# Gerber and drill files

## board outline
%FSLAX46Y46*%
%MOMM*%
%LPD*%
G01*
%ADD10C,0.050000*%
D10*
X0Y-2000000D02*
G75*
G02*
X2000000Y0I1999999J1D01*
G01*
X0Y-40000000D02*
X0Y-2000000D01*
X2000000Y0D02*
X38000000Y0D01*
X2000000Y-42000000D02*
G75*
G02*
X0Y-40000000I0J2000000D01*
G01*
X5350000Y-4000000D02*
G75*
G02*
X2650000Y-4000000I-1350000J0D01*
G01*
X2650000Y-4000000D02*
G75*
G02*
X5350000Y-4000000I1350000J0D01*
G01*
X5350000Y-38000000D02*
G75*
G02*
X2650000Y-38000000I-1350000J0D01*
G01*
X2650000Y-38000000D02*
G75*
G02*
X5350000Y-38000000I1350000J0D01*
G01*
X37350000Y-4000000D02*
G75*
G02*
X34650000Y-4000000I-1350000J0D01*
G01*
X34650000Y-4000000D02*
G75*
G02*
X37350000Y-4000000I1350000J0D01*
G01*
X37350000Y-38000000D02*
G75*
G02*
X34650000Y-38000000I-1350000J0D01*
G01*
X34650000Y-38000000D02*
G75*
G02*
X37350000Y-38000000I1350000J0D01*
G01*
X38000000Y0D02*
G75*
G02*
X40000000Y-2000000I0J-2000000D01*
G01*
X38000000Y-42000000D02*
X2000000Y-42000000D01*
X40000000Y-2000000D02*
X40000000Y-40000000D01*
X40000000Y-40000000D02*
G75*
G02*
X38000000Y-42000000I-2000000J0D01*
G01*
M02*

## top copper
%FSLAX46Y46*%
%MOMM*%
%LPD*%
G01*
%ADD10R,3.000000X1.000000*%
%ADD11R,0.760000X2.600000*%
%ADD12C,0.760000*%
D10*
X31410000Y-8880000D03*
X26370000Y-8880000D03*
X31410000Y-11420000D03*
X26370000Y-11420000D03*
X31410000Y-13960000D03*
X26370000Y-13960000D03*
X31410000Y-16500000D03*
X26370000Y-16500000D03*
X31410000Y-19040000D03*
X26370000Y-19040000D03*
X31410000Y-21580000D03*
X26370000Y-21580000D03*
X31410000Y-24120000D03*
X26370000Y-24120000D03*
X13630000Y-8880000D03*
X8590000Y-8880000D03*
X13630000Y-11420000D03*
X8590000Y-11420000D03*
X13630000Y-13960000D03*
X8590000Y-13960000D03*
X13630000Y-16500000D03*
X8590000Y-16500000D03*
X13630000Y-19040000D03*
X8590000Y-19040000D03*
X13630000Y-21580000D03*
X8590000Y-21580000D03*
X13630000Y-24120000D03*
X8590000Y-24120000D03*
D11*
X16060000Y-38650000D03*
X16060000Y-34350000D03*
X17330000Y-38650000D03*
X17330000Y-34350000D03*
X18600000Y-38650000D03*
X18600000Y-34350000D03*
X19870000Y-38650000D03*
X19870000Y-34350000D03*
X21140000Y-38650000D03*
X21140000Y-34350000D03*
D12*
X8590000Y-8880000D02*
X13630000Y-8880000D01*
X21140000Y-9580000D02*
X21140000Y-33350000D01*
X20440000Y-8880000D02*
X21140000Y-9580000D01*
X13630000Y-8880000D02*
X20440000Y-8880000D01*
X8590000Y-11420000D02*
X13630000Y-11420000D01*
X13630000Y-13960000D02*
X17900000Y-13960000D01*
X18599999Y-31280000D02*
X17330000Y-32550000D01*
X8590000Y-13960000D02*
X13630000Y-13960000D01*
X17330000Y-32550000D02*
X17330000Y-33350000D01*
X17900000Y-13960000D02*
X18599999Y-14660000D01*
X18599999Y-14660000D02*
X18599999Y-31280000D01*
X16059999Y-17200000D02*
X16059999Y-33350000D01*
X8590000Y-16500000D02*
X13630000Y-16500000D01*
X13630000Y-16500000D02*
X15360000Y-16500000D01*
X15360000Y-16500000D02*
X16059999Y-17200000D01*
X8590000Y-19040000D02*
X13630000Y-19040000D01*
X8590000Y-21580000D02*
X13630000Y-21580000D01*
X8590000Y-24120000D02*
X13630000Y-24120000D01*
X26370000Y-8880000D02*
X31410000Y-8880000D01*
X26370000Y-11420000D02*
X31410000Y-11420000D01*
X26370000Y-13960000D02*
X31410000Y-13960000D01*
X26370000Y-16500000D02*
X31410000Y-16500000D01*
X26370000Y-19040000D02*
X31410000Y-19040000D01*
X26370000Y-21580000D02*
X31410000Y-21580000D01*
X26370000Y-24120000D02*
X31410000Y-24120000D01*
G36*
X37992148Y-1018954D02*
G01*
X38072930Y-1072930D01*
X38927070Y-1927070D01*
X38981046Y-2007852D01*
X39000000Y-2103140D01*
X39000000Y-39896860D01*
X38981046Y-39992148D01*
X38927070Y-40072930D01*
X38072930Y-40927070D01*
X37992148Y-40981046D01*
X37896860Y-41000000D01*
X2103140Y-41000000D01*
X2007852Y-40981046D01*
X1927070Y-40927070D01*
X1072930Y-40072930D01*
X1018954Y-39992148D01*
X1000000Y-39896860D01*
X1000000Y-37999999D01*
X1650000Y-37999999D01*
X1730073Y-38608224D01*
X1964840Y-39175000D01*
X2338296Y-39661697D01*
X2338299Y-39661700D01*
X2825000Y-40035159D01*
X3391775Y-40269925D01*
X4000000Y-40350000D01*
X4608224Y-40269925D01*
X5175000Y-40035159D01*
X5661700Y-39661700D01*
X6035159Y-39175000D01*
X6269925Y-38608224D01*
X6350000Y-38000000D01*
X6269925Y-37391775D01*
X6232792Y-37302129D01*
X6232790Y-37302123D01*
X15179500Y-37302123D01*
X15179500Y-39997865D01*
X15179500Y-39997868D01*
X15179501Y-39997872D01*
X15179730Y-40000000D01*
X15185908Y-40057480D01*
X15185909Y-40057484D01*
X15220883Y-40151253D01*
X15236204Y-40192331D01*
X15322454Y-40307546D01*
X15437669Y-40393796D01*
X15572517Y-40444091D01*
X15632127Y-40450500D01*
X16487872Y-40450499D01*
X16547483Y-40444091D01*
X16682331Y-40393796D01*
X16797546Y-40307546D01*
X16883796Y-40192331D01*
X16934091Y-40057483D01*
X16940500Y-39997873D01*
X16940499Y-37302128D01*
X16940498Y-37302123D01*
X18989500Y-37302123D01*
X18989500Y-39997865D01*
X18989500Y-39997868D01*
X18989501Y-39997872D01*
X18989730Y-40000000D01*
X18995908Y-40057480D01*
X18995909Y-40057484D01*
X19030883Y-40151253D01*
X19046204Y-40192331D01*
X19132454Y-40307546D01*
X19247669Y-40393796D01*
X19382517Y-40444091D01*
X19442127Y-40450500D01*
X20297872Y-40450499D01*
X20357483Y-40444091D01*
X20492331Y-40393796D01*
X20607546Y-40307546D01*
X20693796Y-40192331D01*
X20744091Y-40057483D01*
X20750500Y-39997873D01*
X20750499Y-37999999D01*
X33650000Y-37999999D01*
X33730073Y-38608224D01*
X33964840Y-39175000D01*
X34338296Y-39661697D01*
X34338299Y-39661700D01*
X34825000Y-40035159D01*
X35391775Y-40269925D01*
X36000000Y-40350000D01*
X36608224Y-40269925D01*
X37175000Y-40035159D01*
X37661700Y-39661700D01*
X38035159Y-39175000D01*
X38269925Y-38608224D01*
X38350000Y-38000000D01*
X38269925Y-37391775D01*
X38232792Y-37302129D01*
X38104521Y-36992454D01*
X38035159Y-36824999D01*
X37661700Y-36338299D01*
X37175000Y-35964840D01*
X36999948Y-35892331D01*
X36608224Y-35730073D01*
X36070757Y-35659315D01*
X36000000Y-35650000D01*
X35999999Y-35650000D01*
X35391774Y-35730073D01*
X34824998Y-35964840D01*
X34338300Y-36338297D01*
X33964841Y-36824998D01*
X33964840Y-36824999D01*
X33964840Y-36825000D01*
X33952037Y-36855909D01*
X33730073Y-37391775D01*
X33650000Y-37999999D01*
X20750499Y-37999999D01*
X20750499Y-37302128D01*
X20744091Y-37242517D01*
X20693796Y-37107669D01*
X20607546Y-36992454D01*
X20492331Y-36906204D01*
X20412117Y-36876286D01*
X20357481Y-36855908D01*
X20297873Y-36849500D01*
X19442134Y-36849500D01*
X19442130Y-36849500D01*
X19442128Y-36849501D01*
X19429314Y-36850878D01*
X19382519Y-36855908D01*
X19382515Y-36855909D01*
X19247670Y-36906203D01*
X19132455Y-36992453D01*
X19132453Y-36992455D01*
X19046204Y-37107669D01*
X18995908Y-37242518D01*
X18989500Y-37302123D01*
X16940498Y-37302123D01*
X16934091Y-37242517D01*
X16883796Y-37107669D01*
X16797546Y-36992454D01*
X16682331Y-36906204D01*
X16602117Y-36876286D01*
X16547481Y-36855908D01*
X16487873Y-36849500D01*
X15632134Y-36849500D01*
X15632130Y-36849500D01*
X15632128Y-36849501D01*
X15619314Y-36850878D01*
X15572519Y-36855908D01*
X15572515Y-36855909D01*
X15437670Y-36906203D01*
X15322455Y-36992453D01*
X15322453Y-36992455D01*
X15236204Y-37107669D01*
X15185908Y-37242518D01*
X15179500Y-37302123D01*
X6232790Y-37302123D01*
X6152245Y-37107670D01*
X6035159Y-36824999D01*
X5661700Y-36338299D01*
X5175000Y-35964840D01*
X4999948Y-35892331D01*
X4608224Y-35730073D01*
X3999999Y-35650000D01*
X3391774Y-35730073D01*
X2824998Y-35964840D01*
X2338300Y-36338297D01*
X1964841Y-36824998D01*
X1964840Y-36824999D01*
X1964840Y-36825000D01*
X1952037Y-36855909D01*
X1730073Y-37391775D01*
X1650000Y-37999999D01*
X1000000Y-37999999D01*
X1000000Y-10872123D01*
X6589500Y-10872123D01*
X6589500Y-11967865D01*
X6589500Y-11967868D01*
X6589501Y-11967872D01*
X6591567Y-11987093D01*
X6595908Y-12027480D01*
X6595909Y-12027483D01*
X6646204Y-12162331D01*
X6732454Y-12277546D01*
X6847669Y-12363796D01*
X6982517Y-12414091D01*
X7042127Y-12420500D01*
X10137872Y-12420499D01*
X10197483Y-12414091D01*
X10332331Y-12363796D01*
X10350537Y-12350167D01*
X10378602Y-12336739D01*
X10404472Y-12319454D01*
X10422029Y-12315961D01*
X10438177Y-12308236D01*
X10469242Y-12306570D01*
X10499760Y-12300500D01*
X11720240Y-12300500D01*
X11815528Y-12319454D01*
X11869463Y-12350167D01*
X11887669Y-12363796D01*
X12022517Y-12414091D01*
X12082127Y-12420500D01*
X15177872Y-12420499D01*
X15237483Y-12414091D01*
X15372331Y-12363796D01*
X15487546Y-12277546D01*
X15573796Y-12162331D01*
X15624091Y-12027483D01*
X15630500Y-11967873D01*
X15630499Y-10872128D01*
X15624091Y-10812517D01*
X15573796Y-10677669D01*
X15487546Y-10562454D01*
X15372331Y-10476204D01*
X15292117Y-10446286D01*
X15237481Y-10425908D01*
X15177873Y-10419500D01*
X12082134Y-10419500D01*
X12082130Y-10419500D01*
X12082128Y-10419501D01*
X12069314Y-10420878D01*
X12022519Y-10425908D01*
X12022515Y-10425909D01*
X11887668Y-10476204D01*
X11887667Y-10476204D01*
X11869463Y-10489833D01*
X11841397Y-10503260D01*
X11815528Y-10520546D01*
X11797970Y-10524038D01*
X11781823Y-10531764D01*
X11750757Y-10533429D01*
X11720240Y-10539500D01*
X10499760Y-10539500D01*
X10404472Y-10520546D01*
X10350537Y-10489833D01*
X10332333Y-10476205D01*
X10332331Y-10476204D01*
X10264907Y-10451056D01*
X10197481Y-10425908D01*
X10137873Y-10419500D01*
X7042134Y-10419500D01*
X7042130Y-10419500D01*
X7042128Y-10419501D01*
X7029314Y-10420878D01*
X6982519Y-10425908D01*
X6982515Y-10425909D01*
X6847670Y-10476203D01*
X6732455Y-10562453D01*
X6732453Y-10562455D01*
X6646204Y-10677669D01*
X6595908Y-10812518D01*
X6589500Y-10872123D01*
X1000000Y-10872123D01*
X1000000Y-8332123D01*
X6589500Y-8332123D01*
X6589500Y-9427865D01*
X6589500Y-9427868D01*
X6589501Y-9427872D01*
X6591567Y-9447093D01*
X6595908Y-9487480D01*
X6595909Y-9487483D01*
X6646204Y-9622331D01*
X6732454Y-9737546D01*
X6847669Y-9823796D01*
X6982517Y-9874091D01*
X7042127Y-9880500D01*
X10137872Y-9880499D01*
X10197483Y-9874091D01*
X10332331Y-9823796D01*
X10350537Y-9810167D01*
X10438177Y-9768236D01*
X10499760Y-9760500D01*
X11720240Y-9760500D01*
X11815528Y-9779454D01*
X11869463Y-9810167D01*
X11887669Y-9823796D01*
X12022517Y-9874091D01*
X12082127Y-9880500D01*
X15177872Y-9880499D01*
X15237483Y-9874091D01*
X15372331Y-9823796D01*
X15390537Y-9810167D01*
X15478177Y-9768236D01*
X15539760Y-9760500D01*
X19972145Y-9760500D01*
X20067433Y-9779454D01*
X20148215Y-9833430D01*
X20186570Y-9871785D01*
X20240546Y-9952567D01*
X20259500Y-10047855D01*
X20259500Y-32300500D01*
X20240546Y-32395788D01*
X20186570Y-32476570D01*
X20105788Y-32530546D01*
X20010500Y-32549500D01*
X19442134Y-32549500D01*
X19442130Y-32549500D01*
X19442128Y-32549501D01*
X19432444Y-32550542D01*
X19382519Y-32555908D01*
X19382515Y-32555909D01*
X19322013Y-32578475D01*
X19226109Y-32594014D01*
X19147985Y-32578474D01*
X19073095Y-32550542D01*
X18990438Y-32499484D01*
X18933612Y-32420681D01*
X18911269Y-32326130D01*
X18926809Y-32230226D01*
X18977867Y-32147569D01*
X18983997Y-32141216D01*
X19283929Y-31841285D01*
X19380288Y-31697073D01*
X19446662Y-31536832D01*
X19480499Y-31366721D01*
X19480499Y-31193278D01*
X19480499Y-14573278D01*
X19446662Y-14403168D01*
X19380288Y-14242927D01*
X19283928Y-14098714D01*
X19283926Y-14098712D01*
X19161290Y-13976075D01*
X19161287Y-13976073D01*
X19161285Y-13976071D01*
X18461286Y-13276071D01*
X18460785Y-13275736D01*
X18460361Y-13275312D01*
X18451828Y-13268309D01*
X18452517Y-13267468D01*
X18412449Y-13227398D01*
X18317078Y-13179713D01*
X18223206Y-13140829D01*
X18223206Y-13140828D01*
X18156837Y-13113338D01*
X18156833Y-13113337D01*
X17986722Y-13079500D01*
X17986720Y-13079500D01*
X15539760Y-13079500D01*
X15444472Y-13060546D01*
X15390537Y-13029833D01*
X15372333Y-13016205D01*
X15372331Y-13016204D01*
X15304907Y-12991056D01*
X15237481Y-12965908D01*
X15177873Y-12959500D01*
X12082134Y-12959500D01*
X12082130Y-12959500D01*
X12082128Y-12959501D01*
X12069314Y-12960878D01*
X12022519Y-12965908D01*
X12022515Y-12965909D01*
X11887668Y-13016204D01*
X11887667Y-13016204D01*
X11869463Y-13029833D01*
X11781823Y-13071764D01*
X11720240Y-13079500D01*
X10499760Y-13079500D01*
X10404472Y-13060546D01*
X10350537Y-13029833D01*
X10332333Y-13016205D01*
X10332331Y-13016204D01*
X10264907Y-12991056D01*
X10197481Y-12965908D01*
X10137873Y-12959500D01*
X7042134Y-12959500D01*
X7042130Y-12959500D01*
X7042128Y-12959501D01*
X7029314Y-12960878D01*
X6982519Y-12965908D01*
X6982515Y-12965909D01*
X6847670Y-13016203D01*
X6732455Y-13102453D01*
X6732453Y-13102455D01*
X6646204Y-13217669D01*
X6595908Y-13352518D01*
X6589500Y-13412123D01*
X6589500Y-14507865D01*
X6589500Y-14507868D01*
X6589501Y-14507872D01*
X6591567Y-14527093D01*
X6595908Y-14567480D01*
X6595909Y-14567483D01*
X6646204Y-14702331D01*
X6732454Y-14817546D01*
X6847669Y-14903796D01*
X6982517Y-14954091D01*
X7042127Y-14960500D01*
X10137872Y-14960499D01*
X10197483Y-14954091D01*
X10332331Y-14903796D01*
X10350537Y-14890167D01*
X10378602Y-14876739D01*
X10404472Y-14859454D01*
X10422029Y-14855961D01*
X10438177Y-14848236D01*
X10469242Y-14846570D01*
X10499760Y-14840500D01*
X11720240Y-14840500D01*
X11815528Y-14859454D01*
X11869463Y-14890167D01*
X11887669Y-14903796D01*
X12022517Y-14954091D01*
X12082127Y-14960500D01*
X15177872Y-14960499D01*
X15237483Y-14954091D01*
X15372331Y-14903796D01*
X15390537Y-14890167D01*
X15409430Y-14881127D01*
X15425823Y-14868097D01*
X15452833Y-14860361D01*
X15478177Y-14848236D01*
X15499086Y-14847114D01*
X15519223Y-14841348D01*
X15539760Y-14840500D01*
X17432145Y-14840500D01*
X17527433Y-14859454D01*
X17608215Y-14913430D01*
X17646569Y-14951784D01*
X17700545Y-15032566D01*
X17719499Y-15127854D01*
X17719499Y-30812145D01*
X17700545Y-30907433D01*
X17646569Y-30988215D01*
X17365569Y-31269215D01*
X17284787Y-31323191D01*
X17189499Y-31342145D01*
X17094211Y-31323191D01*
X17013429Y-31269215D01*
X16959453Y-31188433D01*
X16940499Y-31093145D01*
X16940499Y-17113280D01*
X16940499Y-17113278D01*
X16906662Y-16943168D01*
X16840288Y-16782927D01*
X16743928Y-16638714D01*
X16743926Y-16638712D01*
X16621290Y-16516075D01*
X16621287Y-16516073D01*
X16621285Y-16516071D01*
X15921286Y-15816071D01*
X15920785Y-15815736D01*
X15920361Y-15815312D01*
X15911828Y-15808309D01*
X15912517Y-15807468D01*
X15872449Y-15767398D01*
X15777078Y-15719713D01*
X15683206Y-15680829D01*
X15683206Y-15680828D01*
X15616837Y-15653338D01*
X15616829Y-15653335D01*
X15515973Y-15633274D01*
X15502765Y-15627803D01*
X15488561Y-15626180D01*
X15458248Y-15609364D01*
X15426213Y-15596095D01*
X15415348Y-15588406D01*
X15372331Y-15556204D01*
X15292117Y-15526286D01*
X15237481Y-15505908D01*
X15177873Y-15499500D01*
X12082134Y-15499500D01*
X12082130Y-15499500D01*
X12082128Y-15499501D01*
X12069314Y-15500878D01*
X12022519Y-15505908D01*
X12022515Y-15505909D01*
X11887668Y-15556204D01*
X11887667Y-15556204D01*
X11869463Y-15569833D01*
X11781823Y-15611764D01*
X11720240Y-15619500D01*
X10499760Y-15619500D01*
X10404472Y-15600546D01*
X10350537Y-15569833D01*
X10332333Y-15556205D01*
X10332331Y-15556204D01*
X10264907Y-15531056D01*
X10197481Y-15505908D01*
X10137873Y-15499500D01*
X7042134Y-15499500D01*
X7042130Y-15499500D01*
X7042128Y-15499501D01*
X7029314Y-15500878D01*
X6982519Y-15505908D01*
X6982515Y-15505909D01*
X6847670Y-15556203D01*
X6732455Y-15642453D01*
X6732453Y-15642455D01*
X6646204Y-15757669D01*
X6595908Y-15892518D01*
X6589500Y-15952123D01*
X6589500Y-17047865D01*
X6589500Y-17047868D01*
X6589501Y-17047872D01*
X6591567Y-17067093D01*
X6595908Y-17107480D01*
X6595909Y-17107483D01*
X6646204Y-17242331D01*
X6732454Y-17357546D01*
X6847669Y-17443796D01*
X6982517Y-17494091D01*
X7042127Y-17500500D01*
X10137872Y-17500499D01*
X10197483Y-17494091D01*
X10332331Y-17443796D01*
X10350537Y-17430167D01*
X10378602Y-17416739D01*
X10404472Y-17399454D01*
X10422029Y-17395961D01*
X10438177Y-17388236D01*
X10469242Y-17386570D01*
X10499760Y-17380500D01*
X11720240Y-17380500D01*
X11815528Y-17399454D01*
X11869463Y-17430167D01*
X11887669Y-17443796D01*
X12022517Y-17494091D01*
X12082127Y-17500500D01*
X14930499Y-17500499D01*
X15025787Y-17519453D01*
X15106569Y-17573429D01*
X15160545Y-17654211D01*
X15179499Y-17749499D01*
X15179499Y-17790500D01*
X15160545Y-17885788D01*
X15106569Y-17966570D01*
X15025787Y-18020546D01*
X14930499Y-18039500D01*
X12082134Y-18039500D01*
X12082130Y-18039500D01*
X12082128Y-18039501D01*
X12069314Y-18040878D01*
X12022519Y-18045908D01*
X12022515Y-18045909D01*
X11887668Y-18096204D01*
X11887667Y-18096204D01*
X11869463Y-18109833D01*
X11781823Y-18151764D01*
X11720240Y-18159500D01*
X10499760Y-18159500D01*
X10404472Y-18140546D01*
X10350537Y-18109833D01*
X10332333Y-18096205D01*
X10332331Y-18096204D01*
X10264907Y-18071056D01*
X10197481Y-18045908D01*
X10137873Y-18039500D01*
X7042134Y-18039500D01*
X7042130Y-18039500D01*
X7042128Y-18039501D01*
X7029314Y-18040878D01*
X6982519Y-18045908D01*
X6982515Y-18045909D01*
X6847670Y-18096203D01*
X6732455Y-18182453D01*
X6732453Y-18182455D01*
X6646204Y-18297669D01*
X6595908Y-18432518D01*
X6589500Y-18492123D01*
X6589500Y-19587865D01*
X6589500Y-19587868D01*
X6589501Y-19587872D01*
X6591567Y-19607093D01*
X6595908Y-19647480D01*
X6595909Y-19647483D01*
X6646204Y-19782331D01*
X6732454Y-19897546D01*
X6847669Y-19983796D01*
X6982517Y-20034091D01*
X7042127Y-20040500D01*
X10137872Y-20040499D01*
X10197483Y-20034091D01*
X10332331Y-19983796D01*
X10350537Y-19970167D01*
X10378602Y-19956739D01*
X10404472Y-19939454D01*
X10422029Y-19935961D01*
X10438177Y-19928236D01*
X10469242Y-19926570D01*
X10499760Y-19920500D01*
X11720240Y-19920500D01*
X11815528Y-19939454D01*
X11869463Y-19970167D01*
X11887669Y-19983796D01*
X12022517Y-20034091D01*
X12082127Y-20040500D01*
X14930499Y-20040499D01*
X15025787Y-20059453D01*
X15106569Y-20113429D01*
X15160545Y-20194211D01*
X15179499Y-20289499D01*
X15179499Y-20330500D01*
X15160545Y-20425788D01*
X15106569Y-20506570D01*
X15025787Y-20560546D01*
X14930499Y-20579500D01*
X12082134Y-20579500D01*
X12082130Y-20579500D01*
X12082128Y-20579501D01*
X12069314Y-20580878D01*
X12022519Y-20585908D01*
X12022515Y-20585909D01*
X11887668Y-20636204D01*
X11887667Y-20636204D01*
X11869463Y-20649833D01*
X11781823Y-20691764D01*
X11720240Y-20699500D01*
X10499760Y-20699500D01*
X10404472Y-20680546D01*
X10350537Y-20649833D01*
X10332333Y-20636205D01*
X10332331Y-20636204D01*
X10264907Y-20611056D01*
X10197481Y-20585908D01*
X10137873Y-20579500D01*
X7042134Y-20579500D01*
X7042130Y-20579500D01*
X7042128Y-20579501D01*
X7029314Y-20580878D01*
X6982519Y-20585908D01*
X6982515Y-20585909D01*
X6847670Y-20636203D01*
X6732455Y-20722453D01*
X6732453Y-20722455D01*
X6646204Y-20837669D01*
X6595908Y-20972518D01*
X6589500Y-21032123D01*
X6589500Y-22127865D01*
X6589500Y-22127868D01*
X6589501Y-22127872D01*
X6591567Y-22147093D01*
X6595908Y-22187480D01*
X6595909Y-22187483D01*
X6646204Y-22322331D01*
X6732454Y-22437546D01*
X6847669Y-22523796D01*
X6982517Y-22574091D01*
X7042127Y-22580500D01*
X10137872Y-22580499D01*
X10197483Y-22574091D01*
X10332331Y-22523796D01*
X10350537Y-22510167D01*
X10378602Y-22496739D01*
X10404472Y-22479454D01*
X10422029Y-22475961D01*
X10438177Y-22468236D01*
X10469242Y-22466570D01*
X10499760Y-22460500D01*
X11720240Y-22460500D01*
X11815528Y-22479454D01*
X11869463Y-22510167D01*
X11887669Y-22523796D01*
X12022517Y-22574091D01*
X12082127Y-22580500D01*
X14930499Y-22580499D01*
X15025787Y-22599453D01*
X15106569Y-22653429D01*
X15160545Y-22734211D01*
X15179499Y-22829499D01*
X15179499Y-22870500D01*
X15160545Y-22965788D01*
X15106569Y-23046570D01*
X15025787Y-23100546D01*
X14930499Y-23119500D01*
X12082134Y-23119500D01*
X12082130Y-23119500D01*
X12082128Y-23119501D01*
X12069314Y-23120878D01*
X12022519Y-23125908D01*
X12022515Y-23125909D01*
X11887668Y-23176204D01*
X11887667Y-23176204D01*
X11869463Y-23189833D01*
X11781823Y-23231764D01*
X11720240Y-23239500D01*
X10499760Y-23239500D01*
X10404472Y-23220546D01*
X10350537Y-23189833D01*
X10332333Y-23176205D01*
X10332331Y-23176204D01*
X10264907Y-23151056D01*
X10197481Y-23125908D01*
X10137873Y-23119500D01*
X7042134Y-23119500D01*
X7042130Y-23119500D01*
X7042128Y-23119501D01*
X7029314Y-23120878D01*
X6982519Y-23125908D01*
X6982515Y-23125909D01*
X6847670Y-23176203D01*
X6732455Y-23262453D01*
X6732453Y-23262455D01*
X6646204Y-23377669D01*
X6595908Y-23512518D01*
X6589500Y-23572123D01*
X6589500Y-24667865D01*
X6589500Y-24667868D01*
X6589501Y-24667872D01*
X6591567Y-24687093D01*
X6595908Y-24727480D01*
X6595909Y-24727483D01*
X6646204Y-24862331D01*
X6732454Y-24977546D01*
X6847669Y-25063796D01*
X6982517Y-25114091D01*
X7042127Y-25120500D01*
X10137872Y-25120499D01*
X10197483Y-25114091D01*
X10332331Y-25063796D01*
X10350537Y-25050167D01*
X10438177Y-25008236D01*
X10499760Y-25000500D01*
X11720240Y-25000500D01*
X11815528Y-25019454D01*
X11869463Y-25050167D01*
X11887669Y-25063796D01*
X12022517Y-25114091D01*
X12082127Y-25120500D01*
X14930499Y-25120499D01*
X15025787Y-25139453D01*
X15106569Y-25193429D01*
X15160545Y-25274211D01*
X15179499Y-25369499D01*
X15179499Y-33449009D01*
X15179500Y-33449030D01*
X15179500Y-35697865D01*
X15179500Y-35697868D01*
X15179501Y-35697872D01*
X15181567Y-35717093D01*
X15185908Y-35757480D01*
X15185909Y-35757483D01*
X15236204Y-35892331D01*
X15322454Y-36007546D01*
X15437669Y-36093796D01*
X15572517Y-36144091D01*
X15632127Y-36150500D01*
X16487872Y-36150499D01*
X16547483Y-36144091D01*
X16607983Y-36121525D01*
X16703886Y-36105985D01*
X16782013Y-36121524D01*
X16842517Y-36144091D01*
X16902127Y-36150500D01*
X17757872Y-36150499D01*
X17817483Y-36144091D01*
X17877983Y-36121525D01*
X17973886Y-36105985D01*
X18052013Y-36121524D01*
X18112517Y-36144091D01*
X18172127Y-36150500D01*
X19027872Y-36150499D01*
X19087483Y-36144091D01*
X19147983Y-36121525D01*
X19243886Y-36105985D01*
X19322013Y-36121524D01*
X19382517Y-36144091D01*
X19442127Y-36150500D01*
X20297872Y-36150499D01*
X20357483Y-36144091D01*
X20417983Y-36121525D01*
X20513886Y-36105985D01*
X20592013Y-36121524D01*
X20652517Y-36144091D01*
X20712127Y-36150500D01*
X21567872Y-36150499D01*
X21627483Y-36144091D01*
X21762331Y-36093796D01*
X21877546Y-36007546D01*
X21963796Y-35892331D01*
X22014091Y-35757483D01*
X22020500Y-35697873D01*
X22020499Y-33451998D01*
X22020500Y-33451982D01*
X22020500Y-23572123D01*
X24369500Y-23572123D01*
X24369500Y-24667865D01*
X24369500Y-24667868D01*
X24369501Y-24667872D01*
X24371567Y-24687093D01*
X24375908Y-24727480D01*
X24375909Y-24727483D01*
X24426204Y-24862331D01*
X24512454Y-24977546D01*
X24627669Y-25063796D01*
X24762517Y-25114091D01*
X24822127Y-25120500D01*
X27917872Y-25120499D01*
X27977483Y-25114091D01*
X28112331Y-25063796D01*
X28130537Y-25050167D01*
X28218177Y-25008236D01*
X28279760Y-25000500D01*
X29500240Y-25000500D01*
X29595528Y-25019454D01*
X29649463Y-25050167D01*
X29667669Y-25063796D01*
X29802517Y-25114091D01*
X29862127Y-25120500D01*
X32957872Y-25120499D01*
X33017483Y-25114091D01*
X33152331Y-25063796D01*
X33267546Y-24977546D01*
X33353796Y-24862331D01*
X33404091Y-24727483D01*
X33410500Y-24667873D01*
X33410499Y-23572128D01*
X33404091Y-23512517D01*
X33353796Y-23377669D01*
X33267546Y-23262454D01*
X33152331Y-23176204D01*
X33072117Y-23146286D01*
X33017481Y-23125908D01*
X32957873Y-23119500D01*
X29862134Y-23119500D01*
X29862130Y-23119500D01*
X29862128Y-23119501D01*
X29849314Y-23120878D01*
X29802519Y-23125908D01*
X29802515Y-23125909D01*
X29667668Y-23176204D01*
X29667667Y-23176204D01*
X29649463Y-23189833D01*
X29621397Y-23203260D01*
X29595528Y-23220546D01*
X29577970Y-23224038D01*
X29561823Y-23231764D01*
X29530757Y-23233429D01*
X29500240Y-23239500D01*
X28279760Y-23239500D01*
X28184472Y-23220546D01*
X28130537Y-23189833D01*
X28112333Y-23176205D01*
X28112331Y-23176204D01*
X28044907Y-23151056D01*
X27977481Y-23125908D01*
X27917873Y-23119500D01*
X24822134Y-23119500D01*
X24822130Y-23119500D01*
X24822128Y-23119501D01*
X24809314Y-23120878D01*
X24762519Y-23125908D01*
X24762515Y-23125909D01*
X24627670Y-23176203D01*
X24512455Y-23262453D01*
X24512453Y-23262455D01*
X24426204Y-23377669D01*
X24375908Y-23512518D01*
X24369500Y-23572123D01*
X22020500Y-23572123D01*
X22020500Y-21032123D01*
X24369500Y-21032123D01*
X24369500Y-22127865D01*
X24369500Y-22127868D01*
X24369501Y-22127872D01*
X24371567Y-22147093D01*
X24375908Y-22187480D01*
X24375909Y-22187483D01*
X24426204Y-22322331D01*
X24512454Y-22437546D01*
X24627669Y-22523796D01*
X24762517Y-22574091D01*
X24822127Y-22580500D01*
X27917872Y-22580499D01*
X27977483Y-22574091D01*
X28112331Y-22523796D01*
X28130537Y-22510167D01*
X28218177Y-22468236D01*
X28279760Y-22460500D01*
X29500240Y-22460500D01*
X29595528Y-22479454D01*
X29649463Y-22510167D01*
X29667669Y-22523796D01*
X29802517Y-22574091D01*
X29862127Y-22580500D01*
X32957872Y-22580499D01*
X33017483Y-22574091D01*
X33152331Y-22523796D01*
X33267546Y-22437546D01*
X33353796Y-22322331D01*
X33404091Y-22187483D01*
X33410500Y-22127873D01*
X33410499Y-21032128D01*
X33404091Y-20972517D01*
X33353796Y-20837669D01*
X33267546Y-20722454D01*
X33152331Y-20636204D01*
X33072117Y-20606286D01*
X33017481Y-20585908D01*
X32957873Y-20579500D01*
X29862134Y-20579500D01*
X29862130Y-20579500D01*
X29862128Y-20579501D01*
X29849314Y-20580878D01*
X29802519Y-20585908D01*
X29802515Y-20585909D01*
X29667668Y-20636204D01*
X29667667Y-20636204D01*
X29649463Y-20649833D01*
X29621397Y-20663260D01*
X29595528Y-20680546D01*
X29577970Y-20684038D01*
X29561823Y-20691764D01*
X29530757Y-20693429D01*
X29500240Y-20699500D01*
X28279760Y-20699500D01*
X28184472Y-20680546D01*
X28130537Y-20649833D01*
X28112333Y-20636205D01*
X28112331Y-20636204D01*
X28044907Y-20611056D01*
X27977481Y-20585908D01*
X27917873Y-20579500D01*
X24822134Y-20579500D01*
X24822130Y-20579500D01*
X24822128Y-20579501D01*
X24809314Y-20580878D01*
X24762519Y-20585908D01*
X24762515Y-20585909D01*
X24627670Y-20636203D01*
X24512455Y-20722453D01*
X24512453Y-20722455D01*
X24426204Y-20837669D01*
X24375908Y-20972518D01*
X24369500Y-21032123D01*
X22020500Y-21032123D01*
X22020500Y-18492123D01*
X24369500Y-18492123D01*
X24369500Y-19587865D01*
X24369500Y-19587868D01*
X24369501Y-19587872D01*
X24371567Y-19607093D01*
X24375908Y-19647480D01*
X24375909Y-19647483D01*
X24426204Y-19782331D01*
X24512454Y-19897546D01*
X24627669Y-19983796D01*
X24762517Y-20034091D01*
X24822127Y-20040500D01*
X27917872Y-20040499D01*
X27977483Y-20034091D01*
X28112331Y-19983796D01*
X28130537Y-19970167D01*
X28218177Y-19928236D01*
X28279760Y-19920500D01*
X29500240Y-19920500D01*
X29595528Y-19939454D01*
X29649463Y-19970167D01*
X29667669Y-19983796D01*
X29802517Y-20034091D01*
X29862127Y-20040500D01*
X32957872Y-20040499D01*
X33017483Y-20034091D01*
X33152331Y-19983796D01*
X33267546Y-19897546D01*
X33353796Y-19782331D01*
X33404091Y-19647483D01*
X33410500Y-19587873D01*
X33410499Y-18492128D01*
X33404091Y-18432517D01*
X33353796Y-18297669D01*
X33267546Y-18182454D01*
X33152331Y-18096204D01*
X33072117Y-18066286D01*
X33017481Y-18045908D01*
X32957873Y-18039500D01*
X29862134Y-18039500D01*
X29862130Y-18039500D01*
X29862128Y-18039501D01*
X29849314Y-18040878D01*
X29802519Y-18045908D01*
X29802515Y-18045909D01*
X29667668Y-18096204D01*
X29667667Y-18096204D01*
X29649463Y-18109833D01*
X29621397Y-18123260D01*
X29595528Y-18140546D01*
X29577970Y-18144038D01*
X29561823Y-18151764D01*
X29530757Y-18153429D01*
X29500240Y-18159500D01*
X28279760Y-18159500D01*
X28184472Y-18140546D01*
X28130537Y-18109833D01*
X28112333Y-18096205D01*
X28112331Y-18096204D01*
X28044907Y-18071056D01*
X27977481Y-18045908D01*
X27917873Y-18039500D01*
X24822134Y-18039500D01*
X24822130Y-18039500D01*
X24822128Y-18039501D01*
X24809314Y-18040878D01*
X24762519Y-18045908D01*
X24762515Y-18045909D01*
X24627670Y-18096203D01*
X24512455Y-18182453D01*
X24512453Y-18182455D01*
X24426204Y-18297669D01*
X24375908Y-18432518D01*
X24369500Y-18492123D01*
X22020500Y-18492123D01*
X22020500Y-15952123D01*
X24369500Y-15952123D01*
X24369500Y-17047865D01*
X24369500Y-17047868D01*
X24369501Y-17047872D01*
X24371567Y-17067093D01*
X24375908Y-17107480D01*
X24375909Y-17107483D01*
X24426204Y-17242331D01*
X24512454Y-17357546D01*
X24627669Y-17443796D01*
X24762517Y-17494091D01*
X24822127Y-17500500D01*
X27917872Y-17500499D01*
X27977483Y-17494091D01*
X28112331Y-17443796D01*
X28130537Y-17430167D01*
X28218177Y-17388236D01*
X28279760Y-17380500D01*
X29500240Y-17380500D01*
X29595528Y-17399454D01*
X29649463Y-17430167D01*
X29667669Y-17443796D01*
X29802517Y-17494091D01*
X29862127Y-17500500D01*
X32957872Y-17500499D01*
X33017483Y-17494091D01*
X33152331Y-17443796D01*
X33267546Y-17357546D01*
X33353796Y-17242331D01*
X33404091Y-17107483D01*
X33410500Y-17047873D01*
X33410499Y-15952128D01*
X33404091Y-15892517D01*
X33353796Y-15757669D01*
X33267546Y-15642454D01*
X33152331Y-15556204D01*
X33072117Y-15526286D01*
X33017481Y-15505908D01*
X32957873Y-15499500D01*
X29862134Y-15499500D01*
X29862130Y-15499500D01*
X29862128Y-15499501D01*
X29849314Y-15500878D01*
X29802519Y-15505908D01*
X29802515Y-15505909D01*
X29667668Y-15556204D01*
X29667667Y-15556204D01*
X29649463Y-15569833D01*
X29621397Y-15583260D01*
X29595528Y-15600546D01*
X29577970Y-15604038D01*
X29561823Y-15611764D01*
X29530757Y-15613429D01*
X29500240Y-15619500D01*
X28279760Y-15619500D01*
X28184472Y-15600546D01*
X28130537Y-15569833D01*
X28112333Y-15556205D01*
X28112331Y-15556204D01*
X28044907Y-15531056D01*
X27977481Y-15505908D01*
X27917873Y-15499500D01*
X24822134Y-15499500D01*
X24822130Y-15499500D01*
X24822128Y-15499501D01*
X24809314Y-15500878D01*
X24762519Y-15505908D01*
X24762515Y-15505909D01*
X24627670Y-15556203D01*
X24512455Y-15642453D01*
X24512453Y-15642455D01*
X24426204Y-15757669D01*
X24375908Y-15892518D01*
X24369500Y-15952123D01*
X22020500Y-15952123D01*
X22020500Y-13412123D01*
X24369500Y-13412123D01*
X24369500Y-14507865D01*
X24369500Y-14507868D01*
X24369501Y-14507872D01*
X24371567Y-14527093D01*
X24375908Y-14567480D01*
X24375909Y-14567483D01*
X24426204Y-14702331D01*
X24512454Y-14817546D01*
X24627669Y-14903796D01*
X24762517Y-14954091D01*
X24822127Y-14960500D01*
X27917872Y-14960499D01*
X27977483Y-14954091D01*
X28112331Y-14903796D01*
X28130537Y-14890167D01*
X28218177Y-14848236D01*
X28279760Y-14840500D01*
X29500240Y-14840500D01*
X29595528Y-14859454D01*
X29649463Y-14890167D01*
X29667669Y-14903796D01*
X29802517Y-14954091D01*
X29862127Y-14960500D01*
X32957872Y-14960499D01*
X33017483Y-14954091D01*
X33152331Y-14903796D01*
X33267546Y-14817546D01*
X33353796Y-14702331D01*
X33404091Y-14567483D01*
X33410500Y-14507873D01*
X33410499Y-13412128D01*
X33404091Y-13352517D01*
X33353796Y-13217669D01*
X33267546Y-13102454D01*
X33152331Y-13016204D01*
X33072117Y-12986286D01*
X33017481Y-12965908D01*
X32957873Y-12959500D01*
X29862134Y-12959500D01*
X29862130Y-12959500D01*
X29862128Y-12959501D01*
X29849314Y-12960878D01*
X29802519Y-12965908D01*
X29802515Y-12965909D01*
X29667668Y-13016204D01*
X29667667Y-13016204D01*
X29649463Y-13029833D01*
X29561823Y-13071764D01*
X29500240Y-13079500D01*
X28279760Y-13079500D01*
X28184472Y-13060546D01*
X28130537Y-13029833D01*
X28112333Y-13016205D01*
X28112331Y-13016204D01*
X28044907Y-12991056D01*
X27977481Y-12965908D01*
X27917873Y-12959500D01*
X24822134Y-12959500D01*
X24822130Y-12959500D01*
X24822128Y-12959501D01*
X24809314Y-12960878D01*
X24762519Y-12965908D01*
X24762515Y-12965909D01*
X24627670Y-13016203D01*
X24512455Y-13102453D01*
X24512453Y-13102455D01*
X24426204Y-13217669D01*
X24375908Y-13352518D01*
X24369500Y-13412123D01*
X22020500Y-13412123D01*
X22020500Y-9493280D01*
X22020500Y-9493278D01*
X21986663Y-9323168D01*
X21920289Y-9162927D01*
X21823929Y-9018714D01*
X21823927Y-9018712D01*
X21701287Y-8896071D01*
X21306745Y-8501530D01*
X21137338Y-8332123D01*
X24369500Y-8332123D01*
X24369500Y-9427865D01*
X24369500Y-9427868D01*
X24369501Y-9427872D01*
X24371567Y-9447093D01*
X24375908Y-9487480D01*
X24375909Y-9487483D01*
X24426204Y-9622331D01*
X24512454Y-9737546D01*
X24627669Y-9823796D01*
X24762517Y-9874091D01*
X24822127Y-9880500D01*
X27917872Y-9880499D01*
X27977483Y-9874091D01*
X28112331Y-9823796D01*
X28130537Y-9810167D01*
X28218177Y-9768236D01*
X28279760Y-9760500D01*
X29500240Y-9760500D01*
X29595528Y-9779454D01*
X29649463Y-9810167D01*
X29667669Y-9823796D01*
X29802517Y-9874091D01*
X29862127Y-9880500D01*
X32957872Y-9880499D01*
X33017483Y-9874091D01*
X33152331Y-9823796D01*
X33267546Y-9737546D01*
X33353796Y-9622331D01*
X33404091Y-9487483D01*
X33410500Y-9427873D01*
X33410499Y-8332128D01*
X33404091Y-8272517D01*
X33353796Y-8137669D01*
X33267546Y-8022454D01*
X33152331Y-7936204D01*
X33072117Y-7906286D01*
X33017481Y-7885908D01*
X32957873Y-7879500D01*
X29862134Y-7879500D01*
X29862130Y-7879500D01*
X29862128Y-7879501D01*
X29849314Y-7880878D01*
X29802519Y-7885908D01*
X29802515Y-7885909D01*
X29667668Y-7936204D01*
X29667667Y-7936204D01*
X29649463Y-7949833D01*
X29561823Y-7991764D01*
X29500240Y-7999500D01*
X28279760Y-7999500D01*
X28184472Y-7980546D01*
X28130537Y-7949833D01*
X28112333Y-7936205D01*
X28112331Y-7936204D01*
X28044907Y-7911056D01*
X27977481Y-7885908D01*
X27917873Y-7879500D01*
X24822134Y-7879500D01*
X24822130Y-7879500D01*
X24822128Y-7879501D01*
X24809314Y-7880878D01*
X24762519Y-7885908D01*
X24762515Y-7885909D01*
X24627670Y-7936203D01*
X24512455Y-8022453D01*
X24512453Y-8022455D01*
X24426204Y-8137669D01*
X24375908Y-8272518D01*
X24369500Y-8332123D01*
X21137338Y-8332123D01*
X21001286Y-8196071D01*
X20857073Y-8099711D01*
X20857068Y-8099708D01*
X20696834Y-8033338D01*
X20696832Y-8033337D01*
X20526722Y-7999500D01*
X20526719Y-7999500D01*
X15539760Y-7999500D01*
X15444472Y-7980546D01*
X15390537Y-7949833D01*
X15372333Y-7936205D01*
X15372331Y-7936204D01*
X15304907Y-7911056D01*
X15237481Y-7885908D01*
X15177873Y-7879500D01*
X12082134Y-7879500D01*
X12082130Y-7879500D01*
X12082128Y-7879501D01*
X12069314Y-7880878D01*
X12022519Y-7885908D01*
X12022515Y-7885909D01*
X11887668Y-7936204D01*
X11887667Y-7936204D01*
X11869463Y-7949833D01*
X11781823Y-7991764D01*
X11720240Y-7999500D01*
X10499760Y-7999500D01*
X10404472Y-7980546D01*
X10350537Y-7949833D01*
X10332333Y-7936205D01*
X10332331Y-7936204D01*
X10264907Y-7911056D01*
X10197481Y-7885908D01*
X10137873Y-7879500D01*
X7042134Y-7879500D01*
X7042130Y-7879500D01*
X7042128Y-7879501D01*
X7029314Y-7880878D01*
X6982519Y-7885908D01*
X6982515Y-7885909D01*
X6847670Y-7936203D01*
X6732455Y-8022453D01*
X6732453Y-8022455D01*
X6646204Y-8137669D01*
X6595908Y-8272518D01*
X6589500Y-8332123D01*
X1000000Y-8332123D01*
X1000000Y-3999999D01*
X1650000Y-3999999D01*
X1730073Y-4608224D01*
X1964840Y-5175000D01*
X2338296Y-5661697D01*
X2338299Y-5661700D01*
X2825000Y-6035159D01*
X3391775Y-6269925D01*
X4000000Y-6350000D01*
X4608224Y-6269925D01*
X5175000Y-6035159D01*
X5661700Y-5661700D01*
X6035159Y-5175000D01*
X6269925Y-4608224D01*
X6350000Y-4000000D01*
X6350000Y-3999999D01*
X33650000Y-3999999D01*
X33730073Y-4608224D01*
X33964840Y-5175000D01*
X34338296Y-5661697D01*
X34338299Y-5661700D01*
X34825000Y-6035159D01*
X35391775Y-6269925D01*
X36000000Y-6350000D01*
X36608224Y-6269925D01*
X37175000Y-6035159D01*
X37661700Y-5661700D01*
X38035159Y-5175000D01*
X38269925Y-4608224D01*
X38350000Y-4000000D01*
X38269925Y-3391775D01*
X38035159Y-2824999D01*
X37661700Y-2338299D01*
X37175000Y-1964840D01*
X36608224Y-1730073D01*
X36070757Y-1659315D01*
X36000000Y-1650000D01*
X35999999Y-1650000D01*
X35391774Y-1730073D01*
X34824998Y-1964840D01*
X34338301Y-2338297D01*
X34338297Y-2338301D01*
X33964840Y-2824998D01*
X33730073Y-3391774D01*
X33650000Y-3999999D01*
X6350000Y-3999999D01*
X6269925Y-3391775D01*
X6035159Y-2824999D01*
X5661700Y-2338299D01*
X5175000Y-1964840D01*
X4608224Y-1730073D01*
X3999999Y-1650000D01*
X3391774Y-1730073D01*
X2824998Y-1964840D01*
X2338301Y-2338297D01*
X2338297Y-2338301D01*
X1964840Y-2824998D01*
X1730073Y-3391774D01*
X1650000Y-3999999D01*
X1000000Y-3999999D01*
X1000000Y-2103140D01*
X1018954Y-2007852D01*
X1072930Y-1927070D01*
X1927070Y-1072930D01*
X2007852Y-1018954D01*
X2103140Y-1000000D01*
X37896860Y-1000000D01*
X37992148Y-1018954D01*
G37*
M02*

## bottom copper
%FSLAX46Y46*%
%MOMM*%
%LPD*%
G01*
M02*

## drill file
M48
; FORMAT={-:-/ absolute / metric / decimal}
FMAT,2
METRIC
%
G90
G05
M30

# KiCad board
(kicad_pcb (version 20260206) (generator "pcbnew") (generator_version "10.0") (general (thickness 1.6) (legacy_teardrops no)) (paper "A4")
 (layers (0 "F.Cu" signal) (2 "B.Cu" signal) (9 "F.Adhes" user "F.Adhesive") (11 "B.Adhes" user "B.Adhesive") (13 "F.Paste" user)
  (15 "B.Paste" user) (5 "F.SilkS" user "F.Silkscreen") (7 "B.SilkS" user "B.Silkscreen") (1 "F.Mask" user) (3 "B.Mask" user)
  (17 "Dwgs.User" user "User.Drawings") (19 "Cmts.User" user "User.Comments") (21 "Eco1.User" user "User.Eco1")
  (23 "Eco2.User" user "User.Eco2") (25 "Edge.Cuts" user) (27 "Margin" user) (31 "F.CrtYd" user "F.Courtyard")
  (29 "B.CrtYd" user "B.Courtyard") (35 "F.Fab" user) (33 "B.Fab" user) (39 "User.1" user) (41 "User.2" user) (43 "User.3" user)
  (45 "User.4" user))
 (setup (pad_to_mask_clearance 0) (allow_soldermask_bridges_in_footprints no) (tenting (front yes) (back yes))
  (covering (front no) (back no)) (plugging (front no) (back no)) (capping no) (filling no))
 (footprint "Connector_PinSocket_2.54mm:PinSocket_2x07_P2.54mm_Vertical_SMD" (layer "F.Cu") (at 28.89 16.5)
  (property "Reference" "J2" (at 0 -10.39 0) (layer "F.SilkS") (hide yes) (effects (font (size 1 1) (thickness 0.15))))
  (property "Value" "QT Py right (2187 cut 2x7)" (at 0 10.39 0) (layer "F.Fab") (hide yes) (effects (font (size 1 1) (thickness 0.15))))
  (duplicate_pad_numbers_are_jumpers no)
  (pad "1" smd rect (at 2.52 -7.62) (size 3 1) (layers "F.Cu" "F.Mask" "F.Paste") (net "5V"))
  (pad "2" smd rect (at -2.52 -7.62) (size 3 1) (layers "F.Cu" "F.Mask" "F.Paste") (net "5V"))
  (pad "3" smd rect (at 2.52 -5.08) (size 3 1) (layers "F.Cu" "F.Mask" "F.Paste") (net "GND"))
  (pad "4" smd rect (at -2.52 -5.08) (size 3 1) (layers "F.Cu" "F.Mask" "F.Paste") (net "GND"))
  (pad "5" smd rect (at 2.52 -2.54) (size 3 1) (layers "F.Cu" "F.Mask" "F.Paste") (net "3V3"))
  (pad "6" smd rect (at -2.52 -2.54) (size 3 1) (layers "F.Cu" "F.Mask" "F.Paste") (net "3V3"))
  (pad "7" smd rect (at 2.52 0) (size 3 1) (layers "F.Cu" "F.Mask" "F.Paste") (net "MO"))
  (pad "8" smd rect (at -2.52 0) (size 3 1) (layers "F.Cu" "F.Mask" "F.Paste") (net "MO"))
  (pad "9" smd rect (at 2.52 2.54) (size 3 1) (layers "F.Cu" "F.Mask" "F.Paste") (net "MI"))
  (pad "10" smd rect (at -2.52 2.54) (size 3 1) (layers "F.Cu" "F.Mask" "F.Paste") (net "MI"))
  (pad "11" smd rect (at 2.52 5.08) (size 3 1) (layers "F.Cu" "F.Mask" "F.Paste") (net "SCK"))
  (pad "12" smd rect (at -2.52 5.08) (size 3 1) (layers "F.Cu" "F.Mask" "F.Paste") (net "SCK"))
  (pad "13" smd rect (at 2.52 7.62) (size 3 1) (layers "F.Cu" "F.Mask" "F.Paste") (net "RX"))
  (pad "14" smd rect (at -2.52 7.62) (size 3 1) (layers "F.Cu" "F.Mask" "F.Paste") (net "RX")))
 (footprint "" (layer "F.Cu") (at 11.11 26.851)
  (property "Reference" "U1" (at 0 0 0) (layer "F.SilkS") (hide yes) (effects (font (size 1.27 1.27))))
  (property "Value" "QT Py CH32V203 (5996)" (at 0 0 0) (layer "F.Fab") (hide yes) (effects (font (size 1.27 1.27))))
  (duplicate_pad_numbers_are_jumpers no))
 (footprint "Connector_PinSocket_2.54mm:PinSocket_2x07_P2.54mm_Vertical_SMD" (layer "F.Cu") (at 11.11 16.5)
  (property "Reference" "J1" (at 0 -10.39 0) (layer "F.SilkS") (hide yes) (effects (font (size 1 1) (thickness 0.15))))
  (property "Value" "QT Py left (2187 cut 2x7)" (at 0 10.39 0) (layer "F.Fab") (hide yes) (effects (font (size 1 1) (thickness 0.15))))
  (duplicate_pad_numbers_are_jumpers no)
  (pad "1" smd rect (at 2.52 -7.62) (size 3 1) (layers "F.Cu" "F.Mask" "F.Paste") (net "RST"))
  (pad "2" smd rect (at -2.52 -7.62) (size 3 1) (layers "F.Cu" "F.Mask" "F.Paste") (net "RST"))
  (pad "3" smd rect (at 2.52 -5.08) (size 3 1) (layers "F.Cu" "F.Mask" "F.Paste") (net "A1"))
  (pad "4" smd rect (at -2.52 -5.08) (size 3 1) (layers "F.Cu" "F.Mask" "F.Paste") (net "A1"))
  (pad "5" smd rect (at 2.52 -2.54) (size 3 1) (layers "F.Cu" "F.Mask" "F.Paste") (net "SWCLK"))
  (pad "6" smd rect (at -2.52 -2.54) (size 3 1) (layers "F.Cu" "F.Mask" "F.Paste") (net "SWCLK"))
  (pad "7" smd rect (at 2.52 0) (size 3 1) (layers "F.Cu" "F.Mask" "F.Paste") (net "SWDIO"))
  (pad "8" smd rect (at -2.52 0) (size 3 1) (layers "F.Cu" "F.Mask" "F.Paste") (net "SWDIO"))
  (pad "9" smd rect (at 2.52 2.54) (size 3 1) (layers "F.Cu" "F.Mask" "F.Paste") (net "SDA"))
  (pad "10" smd rect (at -2.52 2.54) (size 3 1) (layers "F.Cu" "F.Mask" "F.Paste") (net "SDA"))
  (pad "11" smd rect (at 2.52 5.08) (size 3 1) (layers "F.Cu" "F.Mask" "F.Paste") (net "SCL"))
  (pad "12" smd rect (at -2.52 5.08) (size 3 1) (layers "F.Cu" "F.Mask" "F.Paste") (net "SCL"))
  (pad "13" smd rect (at 2.52 7.62) (size 3 1) (layers "F.Cu" "F.Mask" "F.Paste") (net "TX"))
  (pad "14" smd rect (at -2.52 7.62) (size 3 1) (layers "F.Cu" "F.Mask" "F.Paste") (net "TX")))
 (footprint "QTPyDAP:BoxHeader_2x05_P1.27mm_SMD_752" (layer "F.Cu") (at 18.6 36.5 90)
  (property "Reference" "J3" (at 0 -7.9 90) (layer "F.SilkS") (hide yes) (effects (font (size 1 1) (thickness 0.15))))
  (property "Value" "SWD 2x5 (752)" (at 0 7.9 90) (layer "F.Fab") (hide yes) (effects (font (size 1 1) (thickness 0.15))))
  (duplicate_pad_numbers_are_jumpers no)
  (pad "1" smd rect (at -2.15 -2.54 90) (size 2.6 0.76) (layers "F.Cu" "F.Mask" "F.Paste"))
  (pad "2" smd rect (at 2.15 -2.54 90) (size 2.6 0.76) (layers "F.Cu" "F.Mask" "F.Paste") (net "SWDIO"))
  (pad "3" smd rect (at -2.15 -1.27 90) (size 2.6 0.76) (layers "F.Cu" "F.Mask" "F.Paste") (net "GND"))
  (pad "4" smd rect (at 2.15 -1.27 90) (size 2.6 0.76) (layers "F.Cu" "F.Mask" "F.Paste") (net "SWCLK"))
  (pad "5" smd rect (at -2.15 0 90) (size 2.6 0.76) (layers "F.Cu" "F.Mask" "F.Paste") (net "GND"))
  (pad "6" smd rect (at 2.15 0 90) (size 2.6 0.76) (layers "F.Cu" "F.Mask" "F.Paste"))
  (pad "7" smd rect (at -2.15 1.27 90) (size 2.6 0.76) (layers "F.Cu" "F.Mask" "F.Paste"))
  (pad "8" smd rect (at 2.15 1.27 90) (size 2.6 0.76) (layers "F.Cu" "F.Mask" "F.Paste"))
  (pad "9" smd rect (at -2.15 2.54 90) (size 2.6 0.76) (layers "F.Cu" "F.Mask" "F.Paste") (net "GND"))
  (pad "10" smd rect (at 2.15 2.54 90) (size 2.6 0.76) (layers "F.Cu" "F.Mask" "F.Paste") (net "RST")))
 (gr_arc (start 0 2) (mid 0.585786 0.585786) (end 2 0) (stroke (width 0.05) (type default)) (layer "Edge.Cuts"))
 (gr_line (start 0 40) (end 0 2) (stroke (width 0.05) (type default)) (layer "Edge.Cuts"))
 (gr_line (start 2 0) (end 38 0) (stroke (width 0.05) (type default)) (layer "Edge.Cuts"))
 (gr_arc (start 2 42) (mid 0.585786 41.414213) (end 0 40) (stroke (width 0.05) (type default)) (layer "Edge.Cuts"))
 (gr_circle (center 4 4) (end 5.35 4) (stroke (width 0.05) (type default)) (fill no) (layer "Edge.Cuts"))
 (gr_circle (center 4 38) (end 5.35 38) (stroke (width 0.05) (type default)) (fill no) (layer "Edge.Cuts"))
 (gr_circle (center 36 4) (end 37.35 4) (stroke (width 0.05) (type default)) (fill no) (layer "Edge.Cuts"))
 (gr_circle (center 36 38) (end 37.35 38) (stroke (width 0.05) (type default)) (fill no) (layer "Edge.Cuts"))
 (gr_arc (start 38 0) (mid 39.414213 0.585786) (end 40 2) (stroke (width 0.05) (type default)) (layer "Edge.Cuts"))
 (gr_line (start 38 42) (end 2 42) (stroke (width 0.05) (type default)) (layer "Edge.Cuts"))
 (gr_line (start 40 2) (end 40 40) (stroke (width 0.05) (type default)) (layer "Edge.Cuts"))
 (gr_arc (start 40 40) (mid 39.414213 41.414213) (end 38 42) (stroke (width 0.05) (type default)) (layer "Edge.Cuts"))
 (segment (start 8.59 8.88) (end 13.63 8.88) (width 0.76) (layer "F.Cu") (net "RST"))
 (segment (start 21.14 9.58) (end 21.14 33.35) (width 0.76) (layer "F.Cu") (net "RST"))
 (segment (start 20.44 8.88) (end 21.14 9.58) (width 0.76) (layer "F.Cu") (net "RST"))
 (segment (start 13.63 8.88) (end 20.44 8.88) (width 0.76) (layer "F.Cu") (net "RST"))
 (segment (start 8.59 11.42) (end 13.63 11.42) (width 0.76) (layer "F.Cu") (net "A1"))
 (segment (start 13.63 13.96) (end 17.9 13.96) (width 0.76) (layer "F.Cu") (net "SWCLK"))
 (segment (start 18.599999 31.28) (end 17.33 32.55) (width 0.76) (layer "F.Cu") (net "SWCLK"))
 (segment (start 8.59 13.96) (end 13.63 13.96) (width 0.76) (layer "F.Cu") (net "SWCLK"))
 (segment (start 17.33 32.55) (end 17.33 33.35) (width 0.76) (layer "F.Cu") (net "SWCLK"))
 (segment (start 17.9 13.96) (end 18.599999 14.66) (width 0.76) (layer "F.Cu") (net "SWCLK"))
 (segment (start 18.599999 14.66) (end 18.599999 31.28) (width 0.76) (layer "F.Cu") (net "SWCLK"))
 (segment (start 16.059999 17.2) (end 16.059999 33.35) (width 0.76) (layer "F.Cu") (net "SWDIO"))
 (segment (start 8.59 16.5) (end 13.63 16.5) (width 0.76) (layer "F.Cu") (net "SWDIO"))
 (segment (start 13.63 16.5) (end 15.36 16.5) (width 0.76) (layer "F.Cu") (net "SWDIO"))
 (segment (start 15.36 16.5) (end 16.059999 17.2) (width 0.76) (layer "F.Cu") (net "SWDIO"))
 (segment (start 8.59 19.04) (end 13.63 19.04) (width 0.76) (layer "F.Cu") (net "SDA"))
 (segment (start 8.59 21.58) (end 13.63 21.58) (width 0.76) (layer "F.Cu") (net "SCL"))
 (segment (start 8.59 24.12) (end 13.63 24.12) (width 0.76) (layer "F.Cu") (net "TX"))
 (segment (start 26.37 8.88) (end 31.41 8.88) (width 0.76) (layer "F.Cu") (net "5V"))
 (segment (start 26.37 11.42) (end 31.41 11.42) (width 0.76) (layer "F.Cu") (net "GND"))
 (segment (start 26.37 13.96) (end 31.41 13.96) (width 0.76) (layer "F.Cu") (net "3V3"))
 (segment (start 26.37 16.5) (end 31.41 16.5) (width 0.76) (layer "F.Cu") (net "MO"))
 (segment (start 26.37 19.04) (end 31.41 19.04) (width 0.76) (layer "F.Cu") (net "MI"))
 (segment (start 26.37 21.58) (end 31.41 21.58) (width 0.76) (layer "F.Cu") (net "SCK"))
 (segment (start 26.37 24.12) (end 31.41 24.12) (width 0.76) (layer "F.Cu") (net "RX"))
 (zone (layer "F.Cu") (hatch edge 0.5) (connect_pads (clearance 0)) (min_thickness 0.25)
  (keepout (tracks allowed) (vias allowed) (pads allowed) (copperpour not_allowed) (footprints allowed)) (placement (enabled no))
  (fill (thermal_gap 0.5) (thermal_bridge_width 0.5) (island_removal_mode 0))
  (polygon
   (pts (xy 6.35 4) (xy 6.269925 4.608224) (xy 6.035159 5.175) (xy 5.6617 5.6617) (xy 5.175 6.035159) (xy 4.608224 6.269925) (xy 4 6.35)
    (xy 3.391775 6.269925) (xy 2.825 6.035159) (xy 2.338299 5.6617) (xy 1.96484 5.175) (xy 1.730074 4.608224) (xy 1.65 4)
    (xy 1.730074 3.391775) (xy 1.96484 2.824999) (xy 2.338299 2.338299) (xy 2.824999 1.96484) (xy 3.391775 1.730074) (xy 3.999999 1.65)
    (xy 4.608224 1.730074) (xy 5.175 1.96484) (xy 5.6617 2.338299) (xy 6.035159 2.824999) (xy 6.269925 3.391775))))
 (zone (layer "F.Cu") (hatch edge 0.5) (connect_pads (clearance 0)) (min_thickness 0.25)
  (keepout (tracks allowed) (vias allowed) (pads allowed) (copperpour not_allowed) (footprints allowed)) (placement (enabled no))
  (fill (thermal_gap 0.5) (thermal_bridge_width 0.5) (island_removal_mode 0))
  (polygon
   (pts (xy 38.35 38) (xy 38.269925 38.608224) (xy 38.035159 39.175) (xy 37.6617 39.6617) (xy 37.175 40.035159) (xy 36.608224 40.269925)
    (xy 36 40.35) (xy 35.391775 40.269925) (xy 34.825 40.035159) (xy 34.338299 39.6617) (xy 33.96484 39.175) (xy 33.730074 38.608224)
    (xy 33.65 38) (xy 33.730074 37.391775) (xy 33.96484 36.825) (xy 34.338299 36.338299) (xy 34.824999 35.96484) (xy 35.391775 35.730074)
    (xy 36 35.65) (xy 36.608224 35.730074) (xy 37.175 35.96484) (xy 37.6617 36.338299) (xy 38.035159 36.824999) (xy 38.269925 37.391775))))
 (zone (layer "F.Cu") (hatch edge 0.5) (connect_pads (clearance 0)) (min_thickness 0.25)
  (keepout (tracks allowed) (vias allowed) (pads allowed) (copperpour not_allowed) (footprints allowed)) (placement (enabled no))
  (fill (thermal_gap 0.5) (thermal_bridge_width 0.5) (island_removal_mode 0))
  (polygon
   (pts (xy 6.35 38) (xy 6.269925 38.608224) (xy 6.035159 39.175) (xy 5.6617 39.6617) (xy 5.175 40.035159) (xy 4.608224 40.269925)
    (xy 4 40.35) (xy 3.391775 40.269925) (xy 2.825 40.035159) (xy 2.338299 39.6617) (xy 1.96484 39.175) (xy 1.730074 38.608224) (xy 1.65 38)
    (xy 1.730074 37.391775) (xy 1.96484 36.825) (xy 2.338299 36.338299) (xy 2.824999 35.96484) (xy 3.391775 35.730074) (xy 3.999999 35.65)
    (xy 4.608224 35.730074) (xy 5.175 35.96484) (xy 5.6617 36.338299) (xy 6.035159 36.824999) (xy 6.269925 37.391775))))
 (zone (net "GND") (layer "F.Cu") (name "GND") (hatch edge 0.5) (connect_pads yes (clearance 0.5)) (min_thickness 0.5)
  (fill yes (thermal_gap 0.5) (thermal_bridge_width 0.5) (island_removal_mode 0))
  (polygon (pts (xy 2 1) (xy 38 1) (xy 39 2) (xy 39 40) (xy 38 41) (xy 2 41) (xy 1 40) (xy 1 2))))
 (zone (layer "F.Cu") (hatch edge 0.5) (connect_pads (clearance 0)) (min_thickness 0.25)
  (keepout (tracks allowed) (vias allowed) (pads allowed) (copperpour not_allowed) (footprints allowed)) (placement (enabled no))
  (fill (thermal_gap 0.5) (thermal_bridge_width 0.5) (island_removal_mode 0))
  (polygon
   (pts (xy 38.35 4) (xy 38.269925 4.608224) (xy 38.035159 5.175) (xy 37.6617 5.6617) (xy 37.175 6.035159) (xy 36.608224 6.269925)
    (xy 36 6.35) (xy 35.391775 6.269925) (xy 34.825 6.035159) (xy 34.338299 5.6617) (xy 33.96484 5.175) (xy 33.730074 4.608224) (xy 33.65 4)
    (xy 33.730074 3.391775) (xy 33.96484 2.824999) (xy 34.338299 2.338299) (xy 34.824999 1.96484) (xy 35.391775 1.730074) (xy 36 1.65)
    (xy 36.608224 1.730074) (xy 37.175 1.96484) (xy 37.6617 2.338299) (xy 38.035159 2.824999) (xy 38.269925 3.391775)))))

